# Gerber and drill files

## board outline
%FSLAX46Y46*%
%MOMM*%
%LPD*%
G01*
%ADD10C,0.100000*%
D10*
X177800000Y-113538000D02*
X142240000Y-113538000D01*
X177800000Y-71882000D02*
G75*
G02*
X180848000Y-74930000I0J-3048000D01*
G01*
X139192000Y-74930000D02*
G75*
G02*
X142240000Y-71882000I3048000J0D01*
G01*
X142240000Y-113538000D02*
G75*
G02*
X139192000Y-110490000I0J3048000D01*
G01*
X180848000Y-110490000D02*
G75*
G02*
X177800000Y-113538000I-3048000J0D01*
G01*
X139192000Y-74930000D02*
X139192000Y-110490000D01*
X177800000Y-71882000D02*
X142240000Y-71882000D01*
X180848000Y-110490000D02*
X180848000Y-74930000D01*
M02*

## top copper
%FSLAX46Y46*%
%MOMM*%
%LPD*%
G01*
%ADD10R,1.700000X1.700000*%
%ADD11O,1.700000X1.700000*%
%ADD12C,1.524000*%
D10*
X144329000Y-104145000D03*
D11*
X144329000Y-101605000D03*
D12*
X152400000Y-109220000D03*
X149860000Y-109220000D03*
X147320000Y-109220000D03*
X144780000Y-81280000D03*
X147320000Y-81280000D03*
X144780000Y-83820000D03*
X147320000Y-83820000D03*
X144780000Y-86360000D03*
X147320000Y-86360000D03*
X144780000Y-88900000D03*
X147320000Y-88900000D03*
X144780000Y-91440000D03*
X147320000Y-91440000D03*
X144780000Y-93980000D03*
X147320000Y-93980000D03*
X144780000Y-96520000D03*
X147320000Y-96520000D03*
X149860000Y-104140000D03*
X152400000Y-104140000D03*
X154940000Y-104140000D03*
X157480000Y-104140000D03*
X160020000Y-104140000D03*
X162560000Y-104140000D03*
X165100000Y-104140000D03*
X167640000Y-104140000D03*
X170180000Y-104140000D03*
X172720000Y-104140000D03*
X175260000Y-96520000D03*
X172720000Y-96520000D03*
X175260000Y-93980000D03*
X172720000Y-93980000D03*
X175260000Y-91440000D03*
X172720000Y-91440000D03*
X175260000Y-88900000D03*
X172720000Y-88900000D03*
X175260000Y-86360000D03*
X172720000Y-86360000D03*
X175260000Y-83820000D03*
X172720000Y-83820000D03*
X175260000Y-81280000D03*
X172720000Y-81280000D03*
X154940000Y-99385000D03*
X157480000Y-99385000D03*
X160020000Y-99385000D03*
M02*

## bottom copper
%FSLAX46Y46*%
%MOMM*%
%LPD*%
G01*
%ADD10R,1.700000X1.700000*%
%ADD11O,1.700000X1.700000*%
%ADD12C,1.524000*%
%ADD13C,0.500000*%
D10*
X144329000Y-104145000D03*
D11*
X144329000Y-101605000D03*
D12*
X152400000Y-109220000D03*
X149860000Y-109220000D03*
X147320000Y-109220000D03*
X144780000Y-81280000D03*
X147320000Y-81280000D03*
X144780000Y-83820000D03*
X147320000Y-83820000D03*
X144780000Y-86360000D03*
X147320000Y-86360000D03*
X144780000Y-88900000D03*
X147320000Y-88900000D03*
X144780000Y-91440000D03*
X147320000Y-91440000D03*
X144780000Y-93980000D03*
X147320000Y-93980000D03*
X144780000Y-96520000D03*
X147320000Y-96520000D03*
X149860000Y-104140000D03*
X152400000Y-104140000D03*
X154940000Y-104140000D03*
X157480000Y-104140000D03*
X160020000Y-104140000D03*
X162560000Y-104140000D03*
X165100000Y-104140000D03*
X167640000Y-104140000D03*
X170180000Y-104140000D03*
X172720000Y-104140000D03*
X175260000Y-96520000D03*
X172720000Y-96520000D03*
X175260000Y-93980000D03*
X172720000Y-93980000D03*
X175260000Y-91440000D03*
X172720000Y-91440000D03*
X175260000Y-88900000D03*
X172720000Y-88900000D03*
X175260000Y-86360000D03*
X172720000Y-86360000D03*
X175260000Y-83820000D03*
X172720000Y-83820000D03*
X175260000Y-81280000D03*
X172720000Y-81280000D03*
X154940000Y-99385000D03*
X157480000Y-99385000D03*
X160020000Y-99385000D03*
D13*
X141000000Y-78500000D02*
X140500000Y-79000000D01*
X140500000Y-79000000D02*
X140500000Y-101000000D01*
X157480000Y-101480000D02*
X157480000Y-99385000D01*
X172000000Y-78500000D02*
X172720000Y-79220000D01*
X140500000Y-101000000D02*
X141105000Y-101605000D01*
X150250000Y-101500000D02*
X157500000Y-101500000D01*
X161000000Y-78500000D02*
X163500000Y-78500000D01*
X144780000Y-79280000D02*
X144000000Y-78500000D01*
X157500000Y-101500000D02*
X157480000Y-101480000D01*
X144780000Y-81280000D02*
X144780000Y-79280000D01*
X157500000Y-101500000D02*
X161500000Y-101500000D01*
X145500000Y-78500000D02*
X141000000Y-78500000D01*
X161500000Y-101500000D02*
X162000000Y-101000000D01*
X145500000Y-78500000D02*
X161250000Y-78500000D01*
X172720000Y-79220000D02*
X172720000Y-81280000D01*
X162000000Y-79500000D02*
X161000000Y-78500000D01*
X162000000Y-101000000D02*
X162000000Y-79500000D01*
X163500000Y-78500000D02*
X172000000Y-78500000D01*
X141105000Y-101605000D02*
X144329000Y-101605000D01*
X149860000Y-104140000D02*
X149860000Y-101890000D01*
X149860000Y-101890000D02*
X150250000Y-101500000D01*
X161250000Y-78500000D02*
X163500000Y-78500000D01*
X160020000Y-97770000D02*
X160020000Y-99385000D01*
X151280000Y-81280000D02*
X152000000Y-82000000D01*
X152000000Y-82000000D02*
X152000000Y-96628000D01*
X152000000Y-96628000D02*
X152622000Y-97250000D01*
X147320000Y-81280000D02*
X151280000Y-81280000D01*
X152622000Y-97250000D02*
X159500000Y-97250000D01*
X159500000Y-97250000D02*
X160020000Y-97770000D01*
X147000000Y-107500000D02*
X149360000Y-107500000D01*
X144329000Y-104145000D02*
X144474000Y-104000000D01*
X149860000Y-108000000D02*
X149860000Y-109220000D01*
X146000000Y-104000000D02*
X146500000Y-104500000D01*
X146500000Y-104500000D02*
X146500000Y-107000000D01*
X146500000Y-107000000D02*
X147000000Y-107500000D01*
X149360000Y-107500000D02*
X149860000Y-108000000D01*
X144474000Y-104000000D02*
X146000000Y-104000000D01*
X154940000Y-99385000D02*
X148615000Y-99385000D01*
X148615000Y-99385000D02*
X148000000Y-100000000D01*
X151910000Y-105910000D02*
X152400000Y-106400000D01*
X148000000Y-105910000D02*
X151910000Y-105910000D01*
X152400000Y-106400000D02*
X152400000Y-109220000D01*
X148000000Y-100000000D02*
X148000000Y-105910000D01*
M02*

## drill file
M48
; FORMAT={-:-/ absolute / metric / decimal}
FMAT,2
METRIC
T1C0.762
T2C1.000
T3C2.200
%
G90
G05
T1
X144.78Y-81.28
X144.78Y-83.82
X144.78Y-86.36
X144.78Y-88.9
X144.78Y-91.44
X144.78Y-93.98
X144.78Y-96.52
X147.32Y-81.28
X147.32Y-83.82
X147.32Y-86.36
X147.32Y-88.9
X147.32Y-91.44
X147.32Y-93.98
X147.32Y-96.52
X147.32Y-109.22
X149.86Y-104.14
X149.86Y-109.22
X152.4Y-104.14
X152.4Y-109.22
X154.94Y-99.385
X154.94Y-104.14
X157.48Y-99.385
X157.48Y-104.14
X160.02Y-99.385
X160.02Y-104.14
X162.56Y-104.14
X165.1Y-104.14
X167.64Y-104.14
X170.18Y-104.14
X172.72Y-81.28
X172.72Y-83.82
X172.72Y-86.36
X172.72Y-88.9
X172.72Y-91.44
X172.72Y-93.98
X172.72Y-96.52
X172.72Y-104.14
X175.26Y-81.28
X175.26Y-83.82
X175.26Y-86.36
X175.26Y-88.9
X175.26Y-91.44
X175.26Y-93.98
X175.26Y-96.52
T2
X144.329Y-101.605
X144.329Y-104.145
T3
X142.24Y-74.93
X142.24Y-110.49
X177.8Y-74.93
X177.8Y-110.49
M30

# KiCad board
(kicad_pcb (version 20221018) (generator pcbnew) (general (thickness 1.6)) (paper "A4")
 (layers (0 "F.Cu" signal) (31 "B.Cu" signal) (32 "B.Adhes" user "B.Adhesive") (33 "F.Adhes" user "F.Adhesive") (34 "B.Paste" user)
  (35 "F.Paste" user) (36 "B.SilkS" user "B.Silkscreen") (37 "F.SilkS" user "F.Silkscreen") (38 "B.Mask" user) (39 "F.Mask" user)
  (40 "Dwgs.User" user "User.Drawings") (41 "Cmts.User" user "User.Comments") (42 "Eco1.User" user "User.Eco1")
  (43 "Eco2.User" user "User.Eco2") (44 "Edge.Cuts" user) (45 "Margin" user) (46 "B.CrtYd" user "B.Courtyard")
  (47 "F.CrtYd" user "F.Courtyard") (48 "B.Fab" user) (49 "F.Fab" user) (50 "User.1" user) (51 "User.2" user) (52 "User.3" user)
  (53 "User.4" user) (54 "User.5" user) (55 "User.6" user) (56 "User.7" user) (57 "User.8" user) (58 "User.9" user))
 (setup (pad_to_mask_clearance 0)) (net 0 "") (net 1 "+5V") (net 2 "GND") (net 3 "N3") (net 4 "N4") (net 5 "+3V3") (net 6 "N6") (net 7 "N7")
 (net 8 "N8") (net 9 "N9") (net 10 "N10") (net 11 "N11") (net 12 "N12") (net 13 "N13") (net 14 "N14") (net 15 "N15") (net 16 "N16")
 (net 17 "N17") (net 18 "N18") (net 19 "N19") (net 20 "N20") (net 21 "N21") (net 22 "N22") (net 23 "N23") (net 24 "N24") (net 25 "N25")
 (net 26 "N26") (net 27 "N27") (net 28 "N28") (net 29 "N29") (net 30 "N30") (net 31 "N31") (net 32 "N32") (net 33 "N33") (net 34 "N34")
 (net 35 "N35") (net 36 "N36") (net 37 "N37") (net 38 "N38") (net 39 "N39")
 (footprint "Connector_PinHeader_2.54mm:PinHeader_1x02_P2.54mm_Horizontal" (layer "F.Cu") (at 144.329 104.145 180)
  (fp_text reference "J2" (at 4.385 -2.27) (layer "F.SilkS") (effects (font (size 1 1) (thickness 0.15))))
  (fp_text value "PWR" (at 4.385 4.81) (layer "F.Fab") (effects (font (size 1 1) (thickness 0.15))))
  (pad "1" thru_hole rect (at 0 0 180) (size 1.7 1.7) (drill 1) (layers "*.Cu" "*.Mask") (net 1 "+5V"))
  (pad "2" thru_hole oval (at 0 2.54 180) (size 1.7 1.7) (drill 1) (layers "*.Cu" "*.Mask") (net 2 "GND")))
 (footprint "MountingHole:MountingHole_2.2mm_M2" (layer "F.Cu") (at 142.24 74.93)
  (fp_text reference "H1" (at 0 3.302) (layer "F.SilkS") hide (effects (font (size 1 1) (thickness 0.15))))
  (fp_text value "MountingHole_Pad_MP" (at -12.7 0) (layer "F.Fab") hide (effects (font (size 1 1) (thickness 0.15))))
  (pad "" np_thru_hole circle (at 0 0) (size 2.2 2.2) (drill 2.2) (layers "*.Cu" "*.Mask")))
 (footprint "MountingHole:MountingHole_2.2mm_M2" (layer "F.Cu") (at 142.24 110.49)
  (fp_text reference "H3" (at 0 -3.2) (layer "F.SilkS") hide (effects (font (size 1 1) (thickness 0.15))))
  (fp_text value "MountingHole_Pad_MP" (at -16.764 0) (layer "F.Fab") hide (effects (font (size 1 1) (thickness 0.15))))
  (pad "" np_thru_hole circle (at 0 0) (size 2.2 2.2) (drill 2.2) (layers "*.Cu" "*.Mask")))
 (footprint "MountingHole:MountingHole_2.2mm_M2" (layer "F.Cu") (at 177.8 110.49)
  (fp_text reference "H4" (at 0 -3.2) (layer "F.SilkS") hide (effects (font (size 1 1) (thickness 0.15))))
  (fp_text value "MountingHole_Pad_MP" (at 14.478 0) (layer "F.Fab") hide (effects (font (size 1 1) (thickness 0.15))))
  (pad "" np_thru_hole circle (at 0 0) (size 2.2 2.2) (drill 2.2) (layers "*.Cu" "*.Mask")))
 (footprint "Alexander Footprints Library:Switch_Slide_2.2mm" (layer "F.Cu") (at 149.86 104.14 180)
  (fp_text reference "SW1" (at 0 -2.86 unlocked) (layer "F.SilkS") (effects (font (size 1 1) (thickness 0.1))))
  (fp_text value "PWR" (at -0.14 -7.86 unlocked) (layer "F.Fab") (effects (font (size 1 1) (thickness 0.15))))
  (pad "1" thru_hole circle (at -2.54 -5.08 180) (size 1.524 1.524) (drill 0.762) (layers "*.Cu" "*.Mask") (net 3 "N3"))
  (pad "2" thru_hole circle (at 0 -5.08 180) (size 1.524 1.524) (drill 0.762) (layers "*.Cu" "*.Mask") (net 1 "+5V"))
  (pad "3" thru_hole circle (at 2.54 -5.08 180) (size 1.524 1.524) (drill 0.762) (layers "*.Cu" "*.Mask") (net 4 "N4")))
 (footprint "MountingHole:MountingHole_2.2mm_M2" (layer "F.Cu") (at 177.8 74.93)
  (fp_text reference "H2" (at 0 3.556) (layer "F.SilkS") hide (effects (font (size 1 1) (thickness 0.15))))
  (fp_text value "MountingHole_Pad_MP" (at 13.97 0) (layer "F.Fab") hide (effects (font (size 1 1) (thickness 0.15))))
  (pad "" np_thru_hole circle (at 0 0) (size 2.2 2.2) (drill 2.2) (layers "*.Cu" "*.Mask")))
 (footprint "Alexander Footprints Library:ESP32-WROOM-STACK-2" (layer "F.Cu") (at 160.02 88.9)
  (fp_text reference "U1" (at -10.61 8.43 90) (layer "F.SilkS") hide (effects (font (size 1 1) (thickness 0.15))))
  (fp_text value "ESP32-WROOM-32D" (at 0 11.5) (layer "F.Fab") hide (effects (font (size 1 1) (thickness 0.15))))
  (pad "1" thru_hole circle (at -15.24 -7.62) (size 1.524 1.524) (drill 0.762) (layers "*.Cu" "*.Mask") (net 2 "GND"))
  (pad "2" thru_hole circle (at -12.7 -7.62) (size 1.524 1.524) (drill 0.762) (layers "*.Cu" "*.Mask") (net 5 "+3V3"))
  (pad "3" thru_hole circle (at -15.24 -5.08) (size 1.524 1.524) (drill 0.762) (layers "*.Cu" "*.Mask") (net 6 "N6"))
  (pad "4" thru_hole circle (at -12.7 -5.08) (size 1.524 1.524) (drill 0.762) (layers "*.Cu" "*.Mask") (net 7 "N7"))
  (pad "5" thru_hole circle (at -15.24 -2.54) (size 1.524 1.524) (drill 0.762) (layers "*.Cu" "*.Mask") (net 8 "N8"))
  (pad "6" thru_hole circle (at -12.7 -2.54) (size 1.524 1.524) (drill 0.762) (layers "*.Cu" "*.Mask") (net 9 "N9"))
  (pad "7" thru_hole circle (at -15.24 0) (size 1.524 1.524) (drill 0.762) (layers "*.Cu" "*.Mask") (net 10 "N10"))
  (pad "8" thru_hole circle (at -12.7 0) (size 1.524 1.524) (drill 0.762) (layers "*.Cu" "*.Mask") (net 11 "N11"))
  (pad "9" thru_hole circle (at -15.24 2.54) (size 1.524 1.524) (drill 0.762) (layers "*.Cu" "*.Mask") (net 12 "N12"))
  (pad "10" thru_hole circle (at -12.7 2.54) (size 1.524 1.524) (drill 0.762) (layers "*.Cu" "*.Mask") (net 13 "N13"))
  (pad "11" thru_hole circle (at -15.24 5.08) (size 1.524 1.524) (drill 0.762) (layers "*.Cu" "*.Mask") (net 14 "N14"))
  (pad "12" thru_hole circle (at -12.7 5.08) (size 1.524 1.524) (drill 0.762) (layers "*.Cu" "*.Mask") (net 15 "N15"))
  (pad "13" thru_hole circle (at -15.24 7.62) (size 1.524 1.524) (drill 0.762) (layers "*.Cu" "*.Mask") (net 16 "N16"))
  (pad "14" thru_hole circle (at -12.7 7.62) (size 1.524 1.524) (drill 0.762) (layers "*.Cu" "*.Mask") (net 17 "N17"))
  (pad "15" thru_hole circle (at -10.16 15.24 90) (size 1.524 1.524) (drill 0.762) (layers "*.Cu" "*.Mask") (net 2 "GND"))
  (pad "16" thru_hole circle (at -7.62 15.24 90) (size 1.524 1.524) (drill 0.762) (layers "*.Cu" "*.Mask") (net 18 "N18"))
  (pad "17" thru_hole circle (at -5.08 15.24 90) (size 1.524 1.524) (drill 0.762) (layers "*.Cu" "*.Mask") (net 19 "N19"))
  (pad "18" thru_hole circle (at -2.54 15.24 90) (size 1.524 1.524) (drill 0.762) (layers "*.Cu" "*.Mask") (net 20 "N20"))
  (pad "19" thru_hole circle (at 0 15.24 90) (size 1.524 1.524) (drill 0.762) (layers "*.Cu" "*.Mask") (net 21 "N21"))
  (pad "20" thru_hole circle (at 2.54 15.24 90) (size 1.524 1.524) (drill 0.762) (layers "*.Cu" "*.Mask") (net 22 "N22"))
  (pad "21" thru_hole circle (at 5.08 15.24 90) (size 1.524 1.524) (drill 0.762) (layers "*.Cu" "*.Mask") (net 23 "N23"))
  (pad "22" thru_hole circle (at 7.62 15.24 90) (size 1.524 1.524) (drill 0.762) (layers "*.Cu" "*.Mask") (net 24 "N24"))
  (pad "23" thru_hole circle (at 10.16 15.24 90) (size 1.524 1.524) (drill 0.762) (layers "*.Cu" "*.Mask") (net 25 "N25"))
  (pad "24" thru_hole circle (at 12.7 15.24 90) (size 1.524 1.524) (drill 0.762) (layers "*.Cu" "*.Mask") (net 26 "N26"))
  (pad "25" thru_hole circle (at 15.24 7.62) (size 1.524 1.524) (drill 0.762) (layers "*.Cu" "*.Mask") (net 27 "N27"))
  (pad "26" thru_hole circle (at 12.7 7.62) (size 1.524 1.524) (drill 0.762) (layers "*.Cu" "*.Mask") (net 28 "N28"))
  (pad "27" thru_hole circle (at 15.24 5.08) (size 1.524 1.524) (drill 0.762) (layers "*.Cu" "*.Mask") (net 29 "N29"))
  (pad "28" thru_hole circle (at 12.7 5.08) (size 1.524 1.524) (drill 0.762) (layers "*.Cu" "*.Mask") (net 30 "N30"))
  (pad "29" thru_hole circle (at 15.24 2.54) (size 1.524 1.524) (drill 0.762) (layers "*.Cu" "*.Mask") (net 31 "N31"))
  (pad "30" thru_hole circle (at 12.7 2.54) (size 1.524 1.524) (drill 0.762) (layers "*.Cu" "*.Mask") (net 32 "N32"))
  (pad "31" thru_hole circle (at 15.24 0) (size 1.524 1.524) (drill 0.762) (layers "*.Cu" "*.Mask") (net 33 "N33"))
  (pad "32" thru_hole circle (at 12.7 0) (size 1.524 1.524) (drill 0.762) (layers "*.Cu" "*.Mask") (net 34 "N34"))
  (pad "33" thru_hole circle (at 15.24 -2.54) (size 1.524 1.524) (drill 0.762) (layers "*.Cu" "*.Mask") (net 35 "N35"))
  (pad "34" thru_hole circle (at 12.7 -2.54) (size 1.524 1.524) (drill 0.762) (layers "*.Cu" "*.Mask") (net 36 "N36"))
  (pad "35" thru_hole circle (at 15.24 -5.08) (size 1.524 1.524) (drill 0.762) (layers "*.Cu" "*.Mask") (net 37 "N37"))
  (pad "36" thru_hole circle (at 12.7 -5.08) (size 1.524 1.524) (drill 0.762) (layers "*.Cu" "*.Mask") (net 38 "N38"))
  (pad "37" thru_hole circle (at 15.24 -7.62) (size 1.524 1.524) (drill 0.762) (layers "*.Cu" "*.Mask") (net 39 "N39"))
  (pad "38" thru_hole circle (at 12.7 -7.62) (size 1.524 1.524) (drill 0.762) (layers "*.Cu" "*.Mask") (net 2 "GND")))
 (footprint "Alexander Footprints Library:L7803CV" (layer "F.Cu") (at 157.48 104.465)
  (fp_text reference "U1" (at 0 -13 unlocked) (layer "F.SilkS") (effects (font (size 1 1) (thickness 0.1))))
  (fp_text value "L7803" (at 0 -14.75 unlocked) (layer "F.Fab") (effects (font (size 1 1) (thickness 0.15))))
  (pad "1" thru_hole circle (at -2.54 -5.08) (size 1.524 1.524) (drill 0.762) (layers "*.Cu" "*.Mask") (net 3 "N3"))
  (pad "2" thru_hole circle (at 0 -5.08) (size 1.524 1.524) (drill 0.762) (layers "*.Cu" "*.Mask") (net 2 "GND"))
  (pad "3" thru_hole circle (at 2.54 -5.08) (size 1.524 1.524) (drill 0.762) (layers "*.Cu" "*.Mask") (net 5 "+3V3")))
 (gr_line (start 177.8 113.538) (end 142.24 113.538) (stroke (width 0.1) (type default)) (layer "Edge.Cuts"))
 (gr_arc (start 177.8 71.882) (mid 179.955261 72.774739) (end 180.848 74.93) (stroke (width 0.1) (type default)) (layer "Edge.Cuts"))
 (gr_arc (start 139.192 74.93) (mid 140.084739 72.774739) (end 142.24 71.882) (stroke (width 0.1) (type default)) (layer "Edge.Cuts"))
 (gr_arc (start 142.24 113.538) (mid 140.084739 112.645261) (end 139.192 110.49) (stroke (width 0.1) (type default)) (layer "Edge.Cuts"))
 (gr_arc (start 180.848 110.49) (mid 179.955261 112.645261) (end 177.8 113.538) (stroke (width 0.1) (type default)) (layer "Edge.Cuts"))
 (gr_line (start 139.192 74.93) (end 139.192 110.49) (stroke (width 0.1) (type default)) (layer "Edge.Cuts"))
 (gr_line (start 177.8 71.882) (end 142.24 71.882) (stroke (width 0.1) (type default)) (layer "Edge.Cuts"))
 (gr_line (start 180.848 110.49) (end 180.848 74.93) (stroke (width 0.1) (type default)) (layer "Edge.Cuts"))
 (segment (start 141 78.5) (end 140.5 79) (width 0.5) (layer "B.Cu") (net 2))
 (segment (start 140.5 79) (end 140.5 101) (width 0.5) (layer "B.Cu") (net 2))
 (segment (start 157.48 101.48) (end 157.48 99.385) (width 0.5) (layer "B.Cu") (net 2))
 (segment (start 172 78.5) (end 172.72 79.22) (width 0.5) (layer "B.Cu") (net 2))
 (segment (start 140.5 101) (end 141.105 101.605) (width 0.5) (layer "B.Cu") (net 2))
 (segment (start 150.25 101.5) (end 157.5 101.5) (width 0.5) (layer "B.Cu") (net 2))
 (segment (start 161 78.5) (end 163.5 78.5) (width 0.5) (layer "B.Cu") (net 2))
 (segment (start 144.78 79.28) (end 144 78.5) (width 0.5) (layer "B.Cu") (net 2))
 (segment (start 157.5 101.5) (end 157.48 101.48) (width 0.5) (layer "B.Cu") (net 2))
 (segment (start 144.78 81.28) (end 144.78 79.28) (width 0.5) (layer "B.Cu") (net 2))
 (segment (start 157.5 101.5) (end 161.5 101.5) (width 0.5) (layer "B.Cu") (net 2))
 (segment (start 145.5 78.5) (end 141 78.5) (width 0.5) (layer "B.Cu") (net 2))
 (segment (start 161.5 101.5) (end 162 101) (width 0.5) (layer "B.Cu") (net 2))
 (segment (start 145.5 78.5) (end 161.25 78.5) (width 0.5) (layer "B.Cu") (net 2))
 (segment (start 172.72 79.22) (end 172.72 81.28) (width 0.5) (layer "B.Cu") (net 2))
 (segment (start 162 79.5) (end 161 78.5) (width 0.5) (layer "B.Cu") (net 2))
 (segment (start 162 101) (end 162 79.5) (width 0.5) (layer "B.Cu") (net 2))
 (segment (start 163.5 78.5) (end 172 78.5) (width 0.5) (layer "B.Cu") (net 2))
 (segment (start 141.105 101.605) (end 144.329 101.605) (width 0.5) (layer "B.Cu") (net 2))
 (segment (start 149.86 104.14) (end 149.86 101.89) (width 0.5) (layer "B.Cu") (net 2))
 (segment (start 149.86 101.89) (end 150.25 101.5) (width 0.5) (layer "B.Cu") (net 2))
 (segment (start 161.25 78.5) (end 163.5 78.5) (width 0.5) (layer "B.Cu") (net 2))
 (segment (start 160.02 97.77) (end 160.02 99.385) (width 0.5) (layer "B.Cu") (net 5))
 (segment (start 151.28 81.28) (end 152 82) (width 0.5) (layer "B.Cu") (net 5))
 (segment (start 152 82) (end 152 96.628) (width 0.5) (layer "B.Cu") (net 5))
 (segment (start 152 96.628) (end 152.622 97.25) (width 0.5) (layer "B.Cu") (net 5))
 (segment (start 147.32 81.28) (end 151.28 81.28) (width 0.5) (layer "B.Cu") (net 5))
 (segment (start 152.622 97.25) (end 159.5 97.25) (width 0.5) (layer "B.Cu") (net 5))
 (segment (start 159.5 97.25) (end 160.02 97.77) (width 0.5) (layer "B.Cu") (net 5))
 (segment (start 147 107.5) (end 149.36 107.5) (width 0.5) (layer "B.Cu") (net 1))
 (segment (start 144.329 104.145) (end 144.474 104) (width 0.5) (layer "B.Cu") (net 1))
 (segment (start 149.86 108) (end 149.86 109.22) (width 0.5) (layer "B.Cu") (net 1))
 (segment (start 146 104) (end 146.5 104.5) (width 0.5) (layer "B.Cu") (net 1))
 (segment (start 146.5 104.5) (end 146.5 107) (width 0.5) (layer "B.Cu") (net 1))
 (segment (start 146.5 107) (end 147 107.5) (width 0.5) (layer "B.Cu") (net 1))
 (segment (start 149.36 107.5) (end 149.86 108) (width 0.5) (layer "B.Cu") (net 1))
 (segment (start 144.474 104) (end 146 104) (width 0.5) (layer "B.Cu") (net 1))
 (segment (start 154.94 99.385) (end 148.615 99.385) (width 0.5) (layer "B.Cu") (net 3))
 (segment (start 148.615 99.385) (end 148 100) (width 0.5) (layer "B.Cu") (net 3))
 (segment (start 151.91 105.91) (end 152.4 106.4) (width 0.5) (layer "B.Cu") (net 3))
 (segment (start 148 105.91) (end 151.91 105.91) (width 0.5) (layer "B.Cu") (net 3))
 (segment (start 152.4 106.4) (end 152.4 109.22) (width 0.5) (layer "B.Cu") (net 3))
 (segment (start 148 100) (end 148 105.91) (width 0.5) (layer "B.Cu") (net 3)))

